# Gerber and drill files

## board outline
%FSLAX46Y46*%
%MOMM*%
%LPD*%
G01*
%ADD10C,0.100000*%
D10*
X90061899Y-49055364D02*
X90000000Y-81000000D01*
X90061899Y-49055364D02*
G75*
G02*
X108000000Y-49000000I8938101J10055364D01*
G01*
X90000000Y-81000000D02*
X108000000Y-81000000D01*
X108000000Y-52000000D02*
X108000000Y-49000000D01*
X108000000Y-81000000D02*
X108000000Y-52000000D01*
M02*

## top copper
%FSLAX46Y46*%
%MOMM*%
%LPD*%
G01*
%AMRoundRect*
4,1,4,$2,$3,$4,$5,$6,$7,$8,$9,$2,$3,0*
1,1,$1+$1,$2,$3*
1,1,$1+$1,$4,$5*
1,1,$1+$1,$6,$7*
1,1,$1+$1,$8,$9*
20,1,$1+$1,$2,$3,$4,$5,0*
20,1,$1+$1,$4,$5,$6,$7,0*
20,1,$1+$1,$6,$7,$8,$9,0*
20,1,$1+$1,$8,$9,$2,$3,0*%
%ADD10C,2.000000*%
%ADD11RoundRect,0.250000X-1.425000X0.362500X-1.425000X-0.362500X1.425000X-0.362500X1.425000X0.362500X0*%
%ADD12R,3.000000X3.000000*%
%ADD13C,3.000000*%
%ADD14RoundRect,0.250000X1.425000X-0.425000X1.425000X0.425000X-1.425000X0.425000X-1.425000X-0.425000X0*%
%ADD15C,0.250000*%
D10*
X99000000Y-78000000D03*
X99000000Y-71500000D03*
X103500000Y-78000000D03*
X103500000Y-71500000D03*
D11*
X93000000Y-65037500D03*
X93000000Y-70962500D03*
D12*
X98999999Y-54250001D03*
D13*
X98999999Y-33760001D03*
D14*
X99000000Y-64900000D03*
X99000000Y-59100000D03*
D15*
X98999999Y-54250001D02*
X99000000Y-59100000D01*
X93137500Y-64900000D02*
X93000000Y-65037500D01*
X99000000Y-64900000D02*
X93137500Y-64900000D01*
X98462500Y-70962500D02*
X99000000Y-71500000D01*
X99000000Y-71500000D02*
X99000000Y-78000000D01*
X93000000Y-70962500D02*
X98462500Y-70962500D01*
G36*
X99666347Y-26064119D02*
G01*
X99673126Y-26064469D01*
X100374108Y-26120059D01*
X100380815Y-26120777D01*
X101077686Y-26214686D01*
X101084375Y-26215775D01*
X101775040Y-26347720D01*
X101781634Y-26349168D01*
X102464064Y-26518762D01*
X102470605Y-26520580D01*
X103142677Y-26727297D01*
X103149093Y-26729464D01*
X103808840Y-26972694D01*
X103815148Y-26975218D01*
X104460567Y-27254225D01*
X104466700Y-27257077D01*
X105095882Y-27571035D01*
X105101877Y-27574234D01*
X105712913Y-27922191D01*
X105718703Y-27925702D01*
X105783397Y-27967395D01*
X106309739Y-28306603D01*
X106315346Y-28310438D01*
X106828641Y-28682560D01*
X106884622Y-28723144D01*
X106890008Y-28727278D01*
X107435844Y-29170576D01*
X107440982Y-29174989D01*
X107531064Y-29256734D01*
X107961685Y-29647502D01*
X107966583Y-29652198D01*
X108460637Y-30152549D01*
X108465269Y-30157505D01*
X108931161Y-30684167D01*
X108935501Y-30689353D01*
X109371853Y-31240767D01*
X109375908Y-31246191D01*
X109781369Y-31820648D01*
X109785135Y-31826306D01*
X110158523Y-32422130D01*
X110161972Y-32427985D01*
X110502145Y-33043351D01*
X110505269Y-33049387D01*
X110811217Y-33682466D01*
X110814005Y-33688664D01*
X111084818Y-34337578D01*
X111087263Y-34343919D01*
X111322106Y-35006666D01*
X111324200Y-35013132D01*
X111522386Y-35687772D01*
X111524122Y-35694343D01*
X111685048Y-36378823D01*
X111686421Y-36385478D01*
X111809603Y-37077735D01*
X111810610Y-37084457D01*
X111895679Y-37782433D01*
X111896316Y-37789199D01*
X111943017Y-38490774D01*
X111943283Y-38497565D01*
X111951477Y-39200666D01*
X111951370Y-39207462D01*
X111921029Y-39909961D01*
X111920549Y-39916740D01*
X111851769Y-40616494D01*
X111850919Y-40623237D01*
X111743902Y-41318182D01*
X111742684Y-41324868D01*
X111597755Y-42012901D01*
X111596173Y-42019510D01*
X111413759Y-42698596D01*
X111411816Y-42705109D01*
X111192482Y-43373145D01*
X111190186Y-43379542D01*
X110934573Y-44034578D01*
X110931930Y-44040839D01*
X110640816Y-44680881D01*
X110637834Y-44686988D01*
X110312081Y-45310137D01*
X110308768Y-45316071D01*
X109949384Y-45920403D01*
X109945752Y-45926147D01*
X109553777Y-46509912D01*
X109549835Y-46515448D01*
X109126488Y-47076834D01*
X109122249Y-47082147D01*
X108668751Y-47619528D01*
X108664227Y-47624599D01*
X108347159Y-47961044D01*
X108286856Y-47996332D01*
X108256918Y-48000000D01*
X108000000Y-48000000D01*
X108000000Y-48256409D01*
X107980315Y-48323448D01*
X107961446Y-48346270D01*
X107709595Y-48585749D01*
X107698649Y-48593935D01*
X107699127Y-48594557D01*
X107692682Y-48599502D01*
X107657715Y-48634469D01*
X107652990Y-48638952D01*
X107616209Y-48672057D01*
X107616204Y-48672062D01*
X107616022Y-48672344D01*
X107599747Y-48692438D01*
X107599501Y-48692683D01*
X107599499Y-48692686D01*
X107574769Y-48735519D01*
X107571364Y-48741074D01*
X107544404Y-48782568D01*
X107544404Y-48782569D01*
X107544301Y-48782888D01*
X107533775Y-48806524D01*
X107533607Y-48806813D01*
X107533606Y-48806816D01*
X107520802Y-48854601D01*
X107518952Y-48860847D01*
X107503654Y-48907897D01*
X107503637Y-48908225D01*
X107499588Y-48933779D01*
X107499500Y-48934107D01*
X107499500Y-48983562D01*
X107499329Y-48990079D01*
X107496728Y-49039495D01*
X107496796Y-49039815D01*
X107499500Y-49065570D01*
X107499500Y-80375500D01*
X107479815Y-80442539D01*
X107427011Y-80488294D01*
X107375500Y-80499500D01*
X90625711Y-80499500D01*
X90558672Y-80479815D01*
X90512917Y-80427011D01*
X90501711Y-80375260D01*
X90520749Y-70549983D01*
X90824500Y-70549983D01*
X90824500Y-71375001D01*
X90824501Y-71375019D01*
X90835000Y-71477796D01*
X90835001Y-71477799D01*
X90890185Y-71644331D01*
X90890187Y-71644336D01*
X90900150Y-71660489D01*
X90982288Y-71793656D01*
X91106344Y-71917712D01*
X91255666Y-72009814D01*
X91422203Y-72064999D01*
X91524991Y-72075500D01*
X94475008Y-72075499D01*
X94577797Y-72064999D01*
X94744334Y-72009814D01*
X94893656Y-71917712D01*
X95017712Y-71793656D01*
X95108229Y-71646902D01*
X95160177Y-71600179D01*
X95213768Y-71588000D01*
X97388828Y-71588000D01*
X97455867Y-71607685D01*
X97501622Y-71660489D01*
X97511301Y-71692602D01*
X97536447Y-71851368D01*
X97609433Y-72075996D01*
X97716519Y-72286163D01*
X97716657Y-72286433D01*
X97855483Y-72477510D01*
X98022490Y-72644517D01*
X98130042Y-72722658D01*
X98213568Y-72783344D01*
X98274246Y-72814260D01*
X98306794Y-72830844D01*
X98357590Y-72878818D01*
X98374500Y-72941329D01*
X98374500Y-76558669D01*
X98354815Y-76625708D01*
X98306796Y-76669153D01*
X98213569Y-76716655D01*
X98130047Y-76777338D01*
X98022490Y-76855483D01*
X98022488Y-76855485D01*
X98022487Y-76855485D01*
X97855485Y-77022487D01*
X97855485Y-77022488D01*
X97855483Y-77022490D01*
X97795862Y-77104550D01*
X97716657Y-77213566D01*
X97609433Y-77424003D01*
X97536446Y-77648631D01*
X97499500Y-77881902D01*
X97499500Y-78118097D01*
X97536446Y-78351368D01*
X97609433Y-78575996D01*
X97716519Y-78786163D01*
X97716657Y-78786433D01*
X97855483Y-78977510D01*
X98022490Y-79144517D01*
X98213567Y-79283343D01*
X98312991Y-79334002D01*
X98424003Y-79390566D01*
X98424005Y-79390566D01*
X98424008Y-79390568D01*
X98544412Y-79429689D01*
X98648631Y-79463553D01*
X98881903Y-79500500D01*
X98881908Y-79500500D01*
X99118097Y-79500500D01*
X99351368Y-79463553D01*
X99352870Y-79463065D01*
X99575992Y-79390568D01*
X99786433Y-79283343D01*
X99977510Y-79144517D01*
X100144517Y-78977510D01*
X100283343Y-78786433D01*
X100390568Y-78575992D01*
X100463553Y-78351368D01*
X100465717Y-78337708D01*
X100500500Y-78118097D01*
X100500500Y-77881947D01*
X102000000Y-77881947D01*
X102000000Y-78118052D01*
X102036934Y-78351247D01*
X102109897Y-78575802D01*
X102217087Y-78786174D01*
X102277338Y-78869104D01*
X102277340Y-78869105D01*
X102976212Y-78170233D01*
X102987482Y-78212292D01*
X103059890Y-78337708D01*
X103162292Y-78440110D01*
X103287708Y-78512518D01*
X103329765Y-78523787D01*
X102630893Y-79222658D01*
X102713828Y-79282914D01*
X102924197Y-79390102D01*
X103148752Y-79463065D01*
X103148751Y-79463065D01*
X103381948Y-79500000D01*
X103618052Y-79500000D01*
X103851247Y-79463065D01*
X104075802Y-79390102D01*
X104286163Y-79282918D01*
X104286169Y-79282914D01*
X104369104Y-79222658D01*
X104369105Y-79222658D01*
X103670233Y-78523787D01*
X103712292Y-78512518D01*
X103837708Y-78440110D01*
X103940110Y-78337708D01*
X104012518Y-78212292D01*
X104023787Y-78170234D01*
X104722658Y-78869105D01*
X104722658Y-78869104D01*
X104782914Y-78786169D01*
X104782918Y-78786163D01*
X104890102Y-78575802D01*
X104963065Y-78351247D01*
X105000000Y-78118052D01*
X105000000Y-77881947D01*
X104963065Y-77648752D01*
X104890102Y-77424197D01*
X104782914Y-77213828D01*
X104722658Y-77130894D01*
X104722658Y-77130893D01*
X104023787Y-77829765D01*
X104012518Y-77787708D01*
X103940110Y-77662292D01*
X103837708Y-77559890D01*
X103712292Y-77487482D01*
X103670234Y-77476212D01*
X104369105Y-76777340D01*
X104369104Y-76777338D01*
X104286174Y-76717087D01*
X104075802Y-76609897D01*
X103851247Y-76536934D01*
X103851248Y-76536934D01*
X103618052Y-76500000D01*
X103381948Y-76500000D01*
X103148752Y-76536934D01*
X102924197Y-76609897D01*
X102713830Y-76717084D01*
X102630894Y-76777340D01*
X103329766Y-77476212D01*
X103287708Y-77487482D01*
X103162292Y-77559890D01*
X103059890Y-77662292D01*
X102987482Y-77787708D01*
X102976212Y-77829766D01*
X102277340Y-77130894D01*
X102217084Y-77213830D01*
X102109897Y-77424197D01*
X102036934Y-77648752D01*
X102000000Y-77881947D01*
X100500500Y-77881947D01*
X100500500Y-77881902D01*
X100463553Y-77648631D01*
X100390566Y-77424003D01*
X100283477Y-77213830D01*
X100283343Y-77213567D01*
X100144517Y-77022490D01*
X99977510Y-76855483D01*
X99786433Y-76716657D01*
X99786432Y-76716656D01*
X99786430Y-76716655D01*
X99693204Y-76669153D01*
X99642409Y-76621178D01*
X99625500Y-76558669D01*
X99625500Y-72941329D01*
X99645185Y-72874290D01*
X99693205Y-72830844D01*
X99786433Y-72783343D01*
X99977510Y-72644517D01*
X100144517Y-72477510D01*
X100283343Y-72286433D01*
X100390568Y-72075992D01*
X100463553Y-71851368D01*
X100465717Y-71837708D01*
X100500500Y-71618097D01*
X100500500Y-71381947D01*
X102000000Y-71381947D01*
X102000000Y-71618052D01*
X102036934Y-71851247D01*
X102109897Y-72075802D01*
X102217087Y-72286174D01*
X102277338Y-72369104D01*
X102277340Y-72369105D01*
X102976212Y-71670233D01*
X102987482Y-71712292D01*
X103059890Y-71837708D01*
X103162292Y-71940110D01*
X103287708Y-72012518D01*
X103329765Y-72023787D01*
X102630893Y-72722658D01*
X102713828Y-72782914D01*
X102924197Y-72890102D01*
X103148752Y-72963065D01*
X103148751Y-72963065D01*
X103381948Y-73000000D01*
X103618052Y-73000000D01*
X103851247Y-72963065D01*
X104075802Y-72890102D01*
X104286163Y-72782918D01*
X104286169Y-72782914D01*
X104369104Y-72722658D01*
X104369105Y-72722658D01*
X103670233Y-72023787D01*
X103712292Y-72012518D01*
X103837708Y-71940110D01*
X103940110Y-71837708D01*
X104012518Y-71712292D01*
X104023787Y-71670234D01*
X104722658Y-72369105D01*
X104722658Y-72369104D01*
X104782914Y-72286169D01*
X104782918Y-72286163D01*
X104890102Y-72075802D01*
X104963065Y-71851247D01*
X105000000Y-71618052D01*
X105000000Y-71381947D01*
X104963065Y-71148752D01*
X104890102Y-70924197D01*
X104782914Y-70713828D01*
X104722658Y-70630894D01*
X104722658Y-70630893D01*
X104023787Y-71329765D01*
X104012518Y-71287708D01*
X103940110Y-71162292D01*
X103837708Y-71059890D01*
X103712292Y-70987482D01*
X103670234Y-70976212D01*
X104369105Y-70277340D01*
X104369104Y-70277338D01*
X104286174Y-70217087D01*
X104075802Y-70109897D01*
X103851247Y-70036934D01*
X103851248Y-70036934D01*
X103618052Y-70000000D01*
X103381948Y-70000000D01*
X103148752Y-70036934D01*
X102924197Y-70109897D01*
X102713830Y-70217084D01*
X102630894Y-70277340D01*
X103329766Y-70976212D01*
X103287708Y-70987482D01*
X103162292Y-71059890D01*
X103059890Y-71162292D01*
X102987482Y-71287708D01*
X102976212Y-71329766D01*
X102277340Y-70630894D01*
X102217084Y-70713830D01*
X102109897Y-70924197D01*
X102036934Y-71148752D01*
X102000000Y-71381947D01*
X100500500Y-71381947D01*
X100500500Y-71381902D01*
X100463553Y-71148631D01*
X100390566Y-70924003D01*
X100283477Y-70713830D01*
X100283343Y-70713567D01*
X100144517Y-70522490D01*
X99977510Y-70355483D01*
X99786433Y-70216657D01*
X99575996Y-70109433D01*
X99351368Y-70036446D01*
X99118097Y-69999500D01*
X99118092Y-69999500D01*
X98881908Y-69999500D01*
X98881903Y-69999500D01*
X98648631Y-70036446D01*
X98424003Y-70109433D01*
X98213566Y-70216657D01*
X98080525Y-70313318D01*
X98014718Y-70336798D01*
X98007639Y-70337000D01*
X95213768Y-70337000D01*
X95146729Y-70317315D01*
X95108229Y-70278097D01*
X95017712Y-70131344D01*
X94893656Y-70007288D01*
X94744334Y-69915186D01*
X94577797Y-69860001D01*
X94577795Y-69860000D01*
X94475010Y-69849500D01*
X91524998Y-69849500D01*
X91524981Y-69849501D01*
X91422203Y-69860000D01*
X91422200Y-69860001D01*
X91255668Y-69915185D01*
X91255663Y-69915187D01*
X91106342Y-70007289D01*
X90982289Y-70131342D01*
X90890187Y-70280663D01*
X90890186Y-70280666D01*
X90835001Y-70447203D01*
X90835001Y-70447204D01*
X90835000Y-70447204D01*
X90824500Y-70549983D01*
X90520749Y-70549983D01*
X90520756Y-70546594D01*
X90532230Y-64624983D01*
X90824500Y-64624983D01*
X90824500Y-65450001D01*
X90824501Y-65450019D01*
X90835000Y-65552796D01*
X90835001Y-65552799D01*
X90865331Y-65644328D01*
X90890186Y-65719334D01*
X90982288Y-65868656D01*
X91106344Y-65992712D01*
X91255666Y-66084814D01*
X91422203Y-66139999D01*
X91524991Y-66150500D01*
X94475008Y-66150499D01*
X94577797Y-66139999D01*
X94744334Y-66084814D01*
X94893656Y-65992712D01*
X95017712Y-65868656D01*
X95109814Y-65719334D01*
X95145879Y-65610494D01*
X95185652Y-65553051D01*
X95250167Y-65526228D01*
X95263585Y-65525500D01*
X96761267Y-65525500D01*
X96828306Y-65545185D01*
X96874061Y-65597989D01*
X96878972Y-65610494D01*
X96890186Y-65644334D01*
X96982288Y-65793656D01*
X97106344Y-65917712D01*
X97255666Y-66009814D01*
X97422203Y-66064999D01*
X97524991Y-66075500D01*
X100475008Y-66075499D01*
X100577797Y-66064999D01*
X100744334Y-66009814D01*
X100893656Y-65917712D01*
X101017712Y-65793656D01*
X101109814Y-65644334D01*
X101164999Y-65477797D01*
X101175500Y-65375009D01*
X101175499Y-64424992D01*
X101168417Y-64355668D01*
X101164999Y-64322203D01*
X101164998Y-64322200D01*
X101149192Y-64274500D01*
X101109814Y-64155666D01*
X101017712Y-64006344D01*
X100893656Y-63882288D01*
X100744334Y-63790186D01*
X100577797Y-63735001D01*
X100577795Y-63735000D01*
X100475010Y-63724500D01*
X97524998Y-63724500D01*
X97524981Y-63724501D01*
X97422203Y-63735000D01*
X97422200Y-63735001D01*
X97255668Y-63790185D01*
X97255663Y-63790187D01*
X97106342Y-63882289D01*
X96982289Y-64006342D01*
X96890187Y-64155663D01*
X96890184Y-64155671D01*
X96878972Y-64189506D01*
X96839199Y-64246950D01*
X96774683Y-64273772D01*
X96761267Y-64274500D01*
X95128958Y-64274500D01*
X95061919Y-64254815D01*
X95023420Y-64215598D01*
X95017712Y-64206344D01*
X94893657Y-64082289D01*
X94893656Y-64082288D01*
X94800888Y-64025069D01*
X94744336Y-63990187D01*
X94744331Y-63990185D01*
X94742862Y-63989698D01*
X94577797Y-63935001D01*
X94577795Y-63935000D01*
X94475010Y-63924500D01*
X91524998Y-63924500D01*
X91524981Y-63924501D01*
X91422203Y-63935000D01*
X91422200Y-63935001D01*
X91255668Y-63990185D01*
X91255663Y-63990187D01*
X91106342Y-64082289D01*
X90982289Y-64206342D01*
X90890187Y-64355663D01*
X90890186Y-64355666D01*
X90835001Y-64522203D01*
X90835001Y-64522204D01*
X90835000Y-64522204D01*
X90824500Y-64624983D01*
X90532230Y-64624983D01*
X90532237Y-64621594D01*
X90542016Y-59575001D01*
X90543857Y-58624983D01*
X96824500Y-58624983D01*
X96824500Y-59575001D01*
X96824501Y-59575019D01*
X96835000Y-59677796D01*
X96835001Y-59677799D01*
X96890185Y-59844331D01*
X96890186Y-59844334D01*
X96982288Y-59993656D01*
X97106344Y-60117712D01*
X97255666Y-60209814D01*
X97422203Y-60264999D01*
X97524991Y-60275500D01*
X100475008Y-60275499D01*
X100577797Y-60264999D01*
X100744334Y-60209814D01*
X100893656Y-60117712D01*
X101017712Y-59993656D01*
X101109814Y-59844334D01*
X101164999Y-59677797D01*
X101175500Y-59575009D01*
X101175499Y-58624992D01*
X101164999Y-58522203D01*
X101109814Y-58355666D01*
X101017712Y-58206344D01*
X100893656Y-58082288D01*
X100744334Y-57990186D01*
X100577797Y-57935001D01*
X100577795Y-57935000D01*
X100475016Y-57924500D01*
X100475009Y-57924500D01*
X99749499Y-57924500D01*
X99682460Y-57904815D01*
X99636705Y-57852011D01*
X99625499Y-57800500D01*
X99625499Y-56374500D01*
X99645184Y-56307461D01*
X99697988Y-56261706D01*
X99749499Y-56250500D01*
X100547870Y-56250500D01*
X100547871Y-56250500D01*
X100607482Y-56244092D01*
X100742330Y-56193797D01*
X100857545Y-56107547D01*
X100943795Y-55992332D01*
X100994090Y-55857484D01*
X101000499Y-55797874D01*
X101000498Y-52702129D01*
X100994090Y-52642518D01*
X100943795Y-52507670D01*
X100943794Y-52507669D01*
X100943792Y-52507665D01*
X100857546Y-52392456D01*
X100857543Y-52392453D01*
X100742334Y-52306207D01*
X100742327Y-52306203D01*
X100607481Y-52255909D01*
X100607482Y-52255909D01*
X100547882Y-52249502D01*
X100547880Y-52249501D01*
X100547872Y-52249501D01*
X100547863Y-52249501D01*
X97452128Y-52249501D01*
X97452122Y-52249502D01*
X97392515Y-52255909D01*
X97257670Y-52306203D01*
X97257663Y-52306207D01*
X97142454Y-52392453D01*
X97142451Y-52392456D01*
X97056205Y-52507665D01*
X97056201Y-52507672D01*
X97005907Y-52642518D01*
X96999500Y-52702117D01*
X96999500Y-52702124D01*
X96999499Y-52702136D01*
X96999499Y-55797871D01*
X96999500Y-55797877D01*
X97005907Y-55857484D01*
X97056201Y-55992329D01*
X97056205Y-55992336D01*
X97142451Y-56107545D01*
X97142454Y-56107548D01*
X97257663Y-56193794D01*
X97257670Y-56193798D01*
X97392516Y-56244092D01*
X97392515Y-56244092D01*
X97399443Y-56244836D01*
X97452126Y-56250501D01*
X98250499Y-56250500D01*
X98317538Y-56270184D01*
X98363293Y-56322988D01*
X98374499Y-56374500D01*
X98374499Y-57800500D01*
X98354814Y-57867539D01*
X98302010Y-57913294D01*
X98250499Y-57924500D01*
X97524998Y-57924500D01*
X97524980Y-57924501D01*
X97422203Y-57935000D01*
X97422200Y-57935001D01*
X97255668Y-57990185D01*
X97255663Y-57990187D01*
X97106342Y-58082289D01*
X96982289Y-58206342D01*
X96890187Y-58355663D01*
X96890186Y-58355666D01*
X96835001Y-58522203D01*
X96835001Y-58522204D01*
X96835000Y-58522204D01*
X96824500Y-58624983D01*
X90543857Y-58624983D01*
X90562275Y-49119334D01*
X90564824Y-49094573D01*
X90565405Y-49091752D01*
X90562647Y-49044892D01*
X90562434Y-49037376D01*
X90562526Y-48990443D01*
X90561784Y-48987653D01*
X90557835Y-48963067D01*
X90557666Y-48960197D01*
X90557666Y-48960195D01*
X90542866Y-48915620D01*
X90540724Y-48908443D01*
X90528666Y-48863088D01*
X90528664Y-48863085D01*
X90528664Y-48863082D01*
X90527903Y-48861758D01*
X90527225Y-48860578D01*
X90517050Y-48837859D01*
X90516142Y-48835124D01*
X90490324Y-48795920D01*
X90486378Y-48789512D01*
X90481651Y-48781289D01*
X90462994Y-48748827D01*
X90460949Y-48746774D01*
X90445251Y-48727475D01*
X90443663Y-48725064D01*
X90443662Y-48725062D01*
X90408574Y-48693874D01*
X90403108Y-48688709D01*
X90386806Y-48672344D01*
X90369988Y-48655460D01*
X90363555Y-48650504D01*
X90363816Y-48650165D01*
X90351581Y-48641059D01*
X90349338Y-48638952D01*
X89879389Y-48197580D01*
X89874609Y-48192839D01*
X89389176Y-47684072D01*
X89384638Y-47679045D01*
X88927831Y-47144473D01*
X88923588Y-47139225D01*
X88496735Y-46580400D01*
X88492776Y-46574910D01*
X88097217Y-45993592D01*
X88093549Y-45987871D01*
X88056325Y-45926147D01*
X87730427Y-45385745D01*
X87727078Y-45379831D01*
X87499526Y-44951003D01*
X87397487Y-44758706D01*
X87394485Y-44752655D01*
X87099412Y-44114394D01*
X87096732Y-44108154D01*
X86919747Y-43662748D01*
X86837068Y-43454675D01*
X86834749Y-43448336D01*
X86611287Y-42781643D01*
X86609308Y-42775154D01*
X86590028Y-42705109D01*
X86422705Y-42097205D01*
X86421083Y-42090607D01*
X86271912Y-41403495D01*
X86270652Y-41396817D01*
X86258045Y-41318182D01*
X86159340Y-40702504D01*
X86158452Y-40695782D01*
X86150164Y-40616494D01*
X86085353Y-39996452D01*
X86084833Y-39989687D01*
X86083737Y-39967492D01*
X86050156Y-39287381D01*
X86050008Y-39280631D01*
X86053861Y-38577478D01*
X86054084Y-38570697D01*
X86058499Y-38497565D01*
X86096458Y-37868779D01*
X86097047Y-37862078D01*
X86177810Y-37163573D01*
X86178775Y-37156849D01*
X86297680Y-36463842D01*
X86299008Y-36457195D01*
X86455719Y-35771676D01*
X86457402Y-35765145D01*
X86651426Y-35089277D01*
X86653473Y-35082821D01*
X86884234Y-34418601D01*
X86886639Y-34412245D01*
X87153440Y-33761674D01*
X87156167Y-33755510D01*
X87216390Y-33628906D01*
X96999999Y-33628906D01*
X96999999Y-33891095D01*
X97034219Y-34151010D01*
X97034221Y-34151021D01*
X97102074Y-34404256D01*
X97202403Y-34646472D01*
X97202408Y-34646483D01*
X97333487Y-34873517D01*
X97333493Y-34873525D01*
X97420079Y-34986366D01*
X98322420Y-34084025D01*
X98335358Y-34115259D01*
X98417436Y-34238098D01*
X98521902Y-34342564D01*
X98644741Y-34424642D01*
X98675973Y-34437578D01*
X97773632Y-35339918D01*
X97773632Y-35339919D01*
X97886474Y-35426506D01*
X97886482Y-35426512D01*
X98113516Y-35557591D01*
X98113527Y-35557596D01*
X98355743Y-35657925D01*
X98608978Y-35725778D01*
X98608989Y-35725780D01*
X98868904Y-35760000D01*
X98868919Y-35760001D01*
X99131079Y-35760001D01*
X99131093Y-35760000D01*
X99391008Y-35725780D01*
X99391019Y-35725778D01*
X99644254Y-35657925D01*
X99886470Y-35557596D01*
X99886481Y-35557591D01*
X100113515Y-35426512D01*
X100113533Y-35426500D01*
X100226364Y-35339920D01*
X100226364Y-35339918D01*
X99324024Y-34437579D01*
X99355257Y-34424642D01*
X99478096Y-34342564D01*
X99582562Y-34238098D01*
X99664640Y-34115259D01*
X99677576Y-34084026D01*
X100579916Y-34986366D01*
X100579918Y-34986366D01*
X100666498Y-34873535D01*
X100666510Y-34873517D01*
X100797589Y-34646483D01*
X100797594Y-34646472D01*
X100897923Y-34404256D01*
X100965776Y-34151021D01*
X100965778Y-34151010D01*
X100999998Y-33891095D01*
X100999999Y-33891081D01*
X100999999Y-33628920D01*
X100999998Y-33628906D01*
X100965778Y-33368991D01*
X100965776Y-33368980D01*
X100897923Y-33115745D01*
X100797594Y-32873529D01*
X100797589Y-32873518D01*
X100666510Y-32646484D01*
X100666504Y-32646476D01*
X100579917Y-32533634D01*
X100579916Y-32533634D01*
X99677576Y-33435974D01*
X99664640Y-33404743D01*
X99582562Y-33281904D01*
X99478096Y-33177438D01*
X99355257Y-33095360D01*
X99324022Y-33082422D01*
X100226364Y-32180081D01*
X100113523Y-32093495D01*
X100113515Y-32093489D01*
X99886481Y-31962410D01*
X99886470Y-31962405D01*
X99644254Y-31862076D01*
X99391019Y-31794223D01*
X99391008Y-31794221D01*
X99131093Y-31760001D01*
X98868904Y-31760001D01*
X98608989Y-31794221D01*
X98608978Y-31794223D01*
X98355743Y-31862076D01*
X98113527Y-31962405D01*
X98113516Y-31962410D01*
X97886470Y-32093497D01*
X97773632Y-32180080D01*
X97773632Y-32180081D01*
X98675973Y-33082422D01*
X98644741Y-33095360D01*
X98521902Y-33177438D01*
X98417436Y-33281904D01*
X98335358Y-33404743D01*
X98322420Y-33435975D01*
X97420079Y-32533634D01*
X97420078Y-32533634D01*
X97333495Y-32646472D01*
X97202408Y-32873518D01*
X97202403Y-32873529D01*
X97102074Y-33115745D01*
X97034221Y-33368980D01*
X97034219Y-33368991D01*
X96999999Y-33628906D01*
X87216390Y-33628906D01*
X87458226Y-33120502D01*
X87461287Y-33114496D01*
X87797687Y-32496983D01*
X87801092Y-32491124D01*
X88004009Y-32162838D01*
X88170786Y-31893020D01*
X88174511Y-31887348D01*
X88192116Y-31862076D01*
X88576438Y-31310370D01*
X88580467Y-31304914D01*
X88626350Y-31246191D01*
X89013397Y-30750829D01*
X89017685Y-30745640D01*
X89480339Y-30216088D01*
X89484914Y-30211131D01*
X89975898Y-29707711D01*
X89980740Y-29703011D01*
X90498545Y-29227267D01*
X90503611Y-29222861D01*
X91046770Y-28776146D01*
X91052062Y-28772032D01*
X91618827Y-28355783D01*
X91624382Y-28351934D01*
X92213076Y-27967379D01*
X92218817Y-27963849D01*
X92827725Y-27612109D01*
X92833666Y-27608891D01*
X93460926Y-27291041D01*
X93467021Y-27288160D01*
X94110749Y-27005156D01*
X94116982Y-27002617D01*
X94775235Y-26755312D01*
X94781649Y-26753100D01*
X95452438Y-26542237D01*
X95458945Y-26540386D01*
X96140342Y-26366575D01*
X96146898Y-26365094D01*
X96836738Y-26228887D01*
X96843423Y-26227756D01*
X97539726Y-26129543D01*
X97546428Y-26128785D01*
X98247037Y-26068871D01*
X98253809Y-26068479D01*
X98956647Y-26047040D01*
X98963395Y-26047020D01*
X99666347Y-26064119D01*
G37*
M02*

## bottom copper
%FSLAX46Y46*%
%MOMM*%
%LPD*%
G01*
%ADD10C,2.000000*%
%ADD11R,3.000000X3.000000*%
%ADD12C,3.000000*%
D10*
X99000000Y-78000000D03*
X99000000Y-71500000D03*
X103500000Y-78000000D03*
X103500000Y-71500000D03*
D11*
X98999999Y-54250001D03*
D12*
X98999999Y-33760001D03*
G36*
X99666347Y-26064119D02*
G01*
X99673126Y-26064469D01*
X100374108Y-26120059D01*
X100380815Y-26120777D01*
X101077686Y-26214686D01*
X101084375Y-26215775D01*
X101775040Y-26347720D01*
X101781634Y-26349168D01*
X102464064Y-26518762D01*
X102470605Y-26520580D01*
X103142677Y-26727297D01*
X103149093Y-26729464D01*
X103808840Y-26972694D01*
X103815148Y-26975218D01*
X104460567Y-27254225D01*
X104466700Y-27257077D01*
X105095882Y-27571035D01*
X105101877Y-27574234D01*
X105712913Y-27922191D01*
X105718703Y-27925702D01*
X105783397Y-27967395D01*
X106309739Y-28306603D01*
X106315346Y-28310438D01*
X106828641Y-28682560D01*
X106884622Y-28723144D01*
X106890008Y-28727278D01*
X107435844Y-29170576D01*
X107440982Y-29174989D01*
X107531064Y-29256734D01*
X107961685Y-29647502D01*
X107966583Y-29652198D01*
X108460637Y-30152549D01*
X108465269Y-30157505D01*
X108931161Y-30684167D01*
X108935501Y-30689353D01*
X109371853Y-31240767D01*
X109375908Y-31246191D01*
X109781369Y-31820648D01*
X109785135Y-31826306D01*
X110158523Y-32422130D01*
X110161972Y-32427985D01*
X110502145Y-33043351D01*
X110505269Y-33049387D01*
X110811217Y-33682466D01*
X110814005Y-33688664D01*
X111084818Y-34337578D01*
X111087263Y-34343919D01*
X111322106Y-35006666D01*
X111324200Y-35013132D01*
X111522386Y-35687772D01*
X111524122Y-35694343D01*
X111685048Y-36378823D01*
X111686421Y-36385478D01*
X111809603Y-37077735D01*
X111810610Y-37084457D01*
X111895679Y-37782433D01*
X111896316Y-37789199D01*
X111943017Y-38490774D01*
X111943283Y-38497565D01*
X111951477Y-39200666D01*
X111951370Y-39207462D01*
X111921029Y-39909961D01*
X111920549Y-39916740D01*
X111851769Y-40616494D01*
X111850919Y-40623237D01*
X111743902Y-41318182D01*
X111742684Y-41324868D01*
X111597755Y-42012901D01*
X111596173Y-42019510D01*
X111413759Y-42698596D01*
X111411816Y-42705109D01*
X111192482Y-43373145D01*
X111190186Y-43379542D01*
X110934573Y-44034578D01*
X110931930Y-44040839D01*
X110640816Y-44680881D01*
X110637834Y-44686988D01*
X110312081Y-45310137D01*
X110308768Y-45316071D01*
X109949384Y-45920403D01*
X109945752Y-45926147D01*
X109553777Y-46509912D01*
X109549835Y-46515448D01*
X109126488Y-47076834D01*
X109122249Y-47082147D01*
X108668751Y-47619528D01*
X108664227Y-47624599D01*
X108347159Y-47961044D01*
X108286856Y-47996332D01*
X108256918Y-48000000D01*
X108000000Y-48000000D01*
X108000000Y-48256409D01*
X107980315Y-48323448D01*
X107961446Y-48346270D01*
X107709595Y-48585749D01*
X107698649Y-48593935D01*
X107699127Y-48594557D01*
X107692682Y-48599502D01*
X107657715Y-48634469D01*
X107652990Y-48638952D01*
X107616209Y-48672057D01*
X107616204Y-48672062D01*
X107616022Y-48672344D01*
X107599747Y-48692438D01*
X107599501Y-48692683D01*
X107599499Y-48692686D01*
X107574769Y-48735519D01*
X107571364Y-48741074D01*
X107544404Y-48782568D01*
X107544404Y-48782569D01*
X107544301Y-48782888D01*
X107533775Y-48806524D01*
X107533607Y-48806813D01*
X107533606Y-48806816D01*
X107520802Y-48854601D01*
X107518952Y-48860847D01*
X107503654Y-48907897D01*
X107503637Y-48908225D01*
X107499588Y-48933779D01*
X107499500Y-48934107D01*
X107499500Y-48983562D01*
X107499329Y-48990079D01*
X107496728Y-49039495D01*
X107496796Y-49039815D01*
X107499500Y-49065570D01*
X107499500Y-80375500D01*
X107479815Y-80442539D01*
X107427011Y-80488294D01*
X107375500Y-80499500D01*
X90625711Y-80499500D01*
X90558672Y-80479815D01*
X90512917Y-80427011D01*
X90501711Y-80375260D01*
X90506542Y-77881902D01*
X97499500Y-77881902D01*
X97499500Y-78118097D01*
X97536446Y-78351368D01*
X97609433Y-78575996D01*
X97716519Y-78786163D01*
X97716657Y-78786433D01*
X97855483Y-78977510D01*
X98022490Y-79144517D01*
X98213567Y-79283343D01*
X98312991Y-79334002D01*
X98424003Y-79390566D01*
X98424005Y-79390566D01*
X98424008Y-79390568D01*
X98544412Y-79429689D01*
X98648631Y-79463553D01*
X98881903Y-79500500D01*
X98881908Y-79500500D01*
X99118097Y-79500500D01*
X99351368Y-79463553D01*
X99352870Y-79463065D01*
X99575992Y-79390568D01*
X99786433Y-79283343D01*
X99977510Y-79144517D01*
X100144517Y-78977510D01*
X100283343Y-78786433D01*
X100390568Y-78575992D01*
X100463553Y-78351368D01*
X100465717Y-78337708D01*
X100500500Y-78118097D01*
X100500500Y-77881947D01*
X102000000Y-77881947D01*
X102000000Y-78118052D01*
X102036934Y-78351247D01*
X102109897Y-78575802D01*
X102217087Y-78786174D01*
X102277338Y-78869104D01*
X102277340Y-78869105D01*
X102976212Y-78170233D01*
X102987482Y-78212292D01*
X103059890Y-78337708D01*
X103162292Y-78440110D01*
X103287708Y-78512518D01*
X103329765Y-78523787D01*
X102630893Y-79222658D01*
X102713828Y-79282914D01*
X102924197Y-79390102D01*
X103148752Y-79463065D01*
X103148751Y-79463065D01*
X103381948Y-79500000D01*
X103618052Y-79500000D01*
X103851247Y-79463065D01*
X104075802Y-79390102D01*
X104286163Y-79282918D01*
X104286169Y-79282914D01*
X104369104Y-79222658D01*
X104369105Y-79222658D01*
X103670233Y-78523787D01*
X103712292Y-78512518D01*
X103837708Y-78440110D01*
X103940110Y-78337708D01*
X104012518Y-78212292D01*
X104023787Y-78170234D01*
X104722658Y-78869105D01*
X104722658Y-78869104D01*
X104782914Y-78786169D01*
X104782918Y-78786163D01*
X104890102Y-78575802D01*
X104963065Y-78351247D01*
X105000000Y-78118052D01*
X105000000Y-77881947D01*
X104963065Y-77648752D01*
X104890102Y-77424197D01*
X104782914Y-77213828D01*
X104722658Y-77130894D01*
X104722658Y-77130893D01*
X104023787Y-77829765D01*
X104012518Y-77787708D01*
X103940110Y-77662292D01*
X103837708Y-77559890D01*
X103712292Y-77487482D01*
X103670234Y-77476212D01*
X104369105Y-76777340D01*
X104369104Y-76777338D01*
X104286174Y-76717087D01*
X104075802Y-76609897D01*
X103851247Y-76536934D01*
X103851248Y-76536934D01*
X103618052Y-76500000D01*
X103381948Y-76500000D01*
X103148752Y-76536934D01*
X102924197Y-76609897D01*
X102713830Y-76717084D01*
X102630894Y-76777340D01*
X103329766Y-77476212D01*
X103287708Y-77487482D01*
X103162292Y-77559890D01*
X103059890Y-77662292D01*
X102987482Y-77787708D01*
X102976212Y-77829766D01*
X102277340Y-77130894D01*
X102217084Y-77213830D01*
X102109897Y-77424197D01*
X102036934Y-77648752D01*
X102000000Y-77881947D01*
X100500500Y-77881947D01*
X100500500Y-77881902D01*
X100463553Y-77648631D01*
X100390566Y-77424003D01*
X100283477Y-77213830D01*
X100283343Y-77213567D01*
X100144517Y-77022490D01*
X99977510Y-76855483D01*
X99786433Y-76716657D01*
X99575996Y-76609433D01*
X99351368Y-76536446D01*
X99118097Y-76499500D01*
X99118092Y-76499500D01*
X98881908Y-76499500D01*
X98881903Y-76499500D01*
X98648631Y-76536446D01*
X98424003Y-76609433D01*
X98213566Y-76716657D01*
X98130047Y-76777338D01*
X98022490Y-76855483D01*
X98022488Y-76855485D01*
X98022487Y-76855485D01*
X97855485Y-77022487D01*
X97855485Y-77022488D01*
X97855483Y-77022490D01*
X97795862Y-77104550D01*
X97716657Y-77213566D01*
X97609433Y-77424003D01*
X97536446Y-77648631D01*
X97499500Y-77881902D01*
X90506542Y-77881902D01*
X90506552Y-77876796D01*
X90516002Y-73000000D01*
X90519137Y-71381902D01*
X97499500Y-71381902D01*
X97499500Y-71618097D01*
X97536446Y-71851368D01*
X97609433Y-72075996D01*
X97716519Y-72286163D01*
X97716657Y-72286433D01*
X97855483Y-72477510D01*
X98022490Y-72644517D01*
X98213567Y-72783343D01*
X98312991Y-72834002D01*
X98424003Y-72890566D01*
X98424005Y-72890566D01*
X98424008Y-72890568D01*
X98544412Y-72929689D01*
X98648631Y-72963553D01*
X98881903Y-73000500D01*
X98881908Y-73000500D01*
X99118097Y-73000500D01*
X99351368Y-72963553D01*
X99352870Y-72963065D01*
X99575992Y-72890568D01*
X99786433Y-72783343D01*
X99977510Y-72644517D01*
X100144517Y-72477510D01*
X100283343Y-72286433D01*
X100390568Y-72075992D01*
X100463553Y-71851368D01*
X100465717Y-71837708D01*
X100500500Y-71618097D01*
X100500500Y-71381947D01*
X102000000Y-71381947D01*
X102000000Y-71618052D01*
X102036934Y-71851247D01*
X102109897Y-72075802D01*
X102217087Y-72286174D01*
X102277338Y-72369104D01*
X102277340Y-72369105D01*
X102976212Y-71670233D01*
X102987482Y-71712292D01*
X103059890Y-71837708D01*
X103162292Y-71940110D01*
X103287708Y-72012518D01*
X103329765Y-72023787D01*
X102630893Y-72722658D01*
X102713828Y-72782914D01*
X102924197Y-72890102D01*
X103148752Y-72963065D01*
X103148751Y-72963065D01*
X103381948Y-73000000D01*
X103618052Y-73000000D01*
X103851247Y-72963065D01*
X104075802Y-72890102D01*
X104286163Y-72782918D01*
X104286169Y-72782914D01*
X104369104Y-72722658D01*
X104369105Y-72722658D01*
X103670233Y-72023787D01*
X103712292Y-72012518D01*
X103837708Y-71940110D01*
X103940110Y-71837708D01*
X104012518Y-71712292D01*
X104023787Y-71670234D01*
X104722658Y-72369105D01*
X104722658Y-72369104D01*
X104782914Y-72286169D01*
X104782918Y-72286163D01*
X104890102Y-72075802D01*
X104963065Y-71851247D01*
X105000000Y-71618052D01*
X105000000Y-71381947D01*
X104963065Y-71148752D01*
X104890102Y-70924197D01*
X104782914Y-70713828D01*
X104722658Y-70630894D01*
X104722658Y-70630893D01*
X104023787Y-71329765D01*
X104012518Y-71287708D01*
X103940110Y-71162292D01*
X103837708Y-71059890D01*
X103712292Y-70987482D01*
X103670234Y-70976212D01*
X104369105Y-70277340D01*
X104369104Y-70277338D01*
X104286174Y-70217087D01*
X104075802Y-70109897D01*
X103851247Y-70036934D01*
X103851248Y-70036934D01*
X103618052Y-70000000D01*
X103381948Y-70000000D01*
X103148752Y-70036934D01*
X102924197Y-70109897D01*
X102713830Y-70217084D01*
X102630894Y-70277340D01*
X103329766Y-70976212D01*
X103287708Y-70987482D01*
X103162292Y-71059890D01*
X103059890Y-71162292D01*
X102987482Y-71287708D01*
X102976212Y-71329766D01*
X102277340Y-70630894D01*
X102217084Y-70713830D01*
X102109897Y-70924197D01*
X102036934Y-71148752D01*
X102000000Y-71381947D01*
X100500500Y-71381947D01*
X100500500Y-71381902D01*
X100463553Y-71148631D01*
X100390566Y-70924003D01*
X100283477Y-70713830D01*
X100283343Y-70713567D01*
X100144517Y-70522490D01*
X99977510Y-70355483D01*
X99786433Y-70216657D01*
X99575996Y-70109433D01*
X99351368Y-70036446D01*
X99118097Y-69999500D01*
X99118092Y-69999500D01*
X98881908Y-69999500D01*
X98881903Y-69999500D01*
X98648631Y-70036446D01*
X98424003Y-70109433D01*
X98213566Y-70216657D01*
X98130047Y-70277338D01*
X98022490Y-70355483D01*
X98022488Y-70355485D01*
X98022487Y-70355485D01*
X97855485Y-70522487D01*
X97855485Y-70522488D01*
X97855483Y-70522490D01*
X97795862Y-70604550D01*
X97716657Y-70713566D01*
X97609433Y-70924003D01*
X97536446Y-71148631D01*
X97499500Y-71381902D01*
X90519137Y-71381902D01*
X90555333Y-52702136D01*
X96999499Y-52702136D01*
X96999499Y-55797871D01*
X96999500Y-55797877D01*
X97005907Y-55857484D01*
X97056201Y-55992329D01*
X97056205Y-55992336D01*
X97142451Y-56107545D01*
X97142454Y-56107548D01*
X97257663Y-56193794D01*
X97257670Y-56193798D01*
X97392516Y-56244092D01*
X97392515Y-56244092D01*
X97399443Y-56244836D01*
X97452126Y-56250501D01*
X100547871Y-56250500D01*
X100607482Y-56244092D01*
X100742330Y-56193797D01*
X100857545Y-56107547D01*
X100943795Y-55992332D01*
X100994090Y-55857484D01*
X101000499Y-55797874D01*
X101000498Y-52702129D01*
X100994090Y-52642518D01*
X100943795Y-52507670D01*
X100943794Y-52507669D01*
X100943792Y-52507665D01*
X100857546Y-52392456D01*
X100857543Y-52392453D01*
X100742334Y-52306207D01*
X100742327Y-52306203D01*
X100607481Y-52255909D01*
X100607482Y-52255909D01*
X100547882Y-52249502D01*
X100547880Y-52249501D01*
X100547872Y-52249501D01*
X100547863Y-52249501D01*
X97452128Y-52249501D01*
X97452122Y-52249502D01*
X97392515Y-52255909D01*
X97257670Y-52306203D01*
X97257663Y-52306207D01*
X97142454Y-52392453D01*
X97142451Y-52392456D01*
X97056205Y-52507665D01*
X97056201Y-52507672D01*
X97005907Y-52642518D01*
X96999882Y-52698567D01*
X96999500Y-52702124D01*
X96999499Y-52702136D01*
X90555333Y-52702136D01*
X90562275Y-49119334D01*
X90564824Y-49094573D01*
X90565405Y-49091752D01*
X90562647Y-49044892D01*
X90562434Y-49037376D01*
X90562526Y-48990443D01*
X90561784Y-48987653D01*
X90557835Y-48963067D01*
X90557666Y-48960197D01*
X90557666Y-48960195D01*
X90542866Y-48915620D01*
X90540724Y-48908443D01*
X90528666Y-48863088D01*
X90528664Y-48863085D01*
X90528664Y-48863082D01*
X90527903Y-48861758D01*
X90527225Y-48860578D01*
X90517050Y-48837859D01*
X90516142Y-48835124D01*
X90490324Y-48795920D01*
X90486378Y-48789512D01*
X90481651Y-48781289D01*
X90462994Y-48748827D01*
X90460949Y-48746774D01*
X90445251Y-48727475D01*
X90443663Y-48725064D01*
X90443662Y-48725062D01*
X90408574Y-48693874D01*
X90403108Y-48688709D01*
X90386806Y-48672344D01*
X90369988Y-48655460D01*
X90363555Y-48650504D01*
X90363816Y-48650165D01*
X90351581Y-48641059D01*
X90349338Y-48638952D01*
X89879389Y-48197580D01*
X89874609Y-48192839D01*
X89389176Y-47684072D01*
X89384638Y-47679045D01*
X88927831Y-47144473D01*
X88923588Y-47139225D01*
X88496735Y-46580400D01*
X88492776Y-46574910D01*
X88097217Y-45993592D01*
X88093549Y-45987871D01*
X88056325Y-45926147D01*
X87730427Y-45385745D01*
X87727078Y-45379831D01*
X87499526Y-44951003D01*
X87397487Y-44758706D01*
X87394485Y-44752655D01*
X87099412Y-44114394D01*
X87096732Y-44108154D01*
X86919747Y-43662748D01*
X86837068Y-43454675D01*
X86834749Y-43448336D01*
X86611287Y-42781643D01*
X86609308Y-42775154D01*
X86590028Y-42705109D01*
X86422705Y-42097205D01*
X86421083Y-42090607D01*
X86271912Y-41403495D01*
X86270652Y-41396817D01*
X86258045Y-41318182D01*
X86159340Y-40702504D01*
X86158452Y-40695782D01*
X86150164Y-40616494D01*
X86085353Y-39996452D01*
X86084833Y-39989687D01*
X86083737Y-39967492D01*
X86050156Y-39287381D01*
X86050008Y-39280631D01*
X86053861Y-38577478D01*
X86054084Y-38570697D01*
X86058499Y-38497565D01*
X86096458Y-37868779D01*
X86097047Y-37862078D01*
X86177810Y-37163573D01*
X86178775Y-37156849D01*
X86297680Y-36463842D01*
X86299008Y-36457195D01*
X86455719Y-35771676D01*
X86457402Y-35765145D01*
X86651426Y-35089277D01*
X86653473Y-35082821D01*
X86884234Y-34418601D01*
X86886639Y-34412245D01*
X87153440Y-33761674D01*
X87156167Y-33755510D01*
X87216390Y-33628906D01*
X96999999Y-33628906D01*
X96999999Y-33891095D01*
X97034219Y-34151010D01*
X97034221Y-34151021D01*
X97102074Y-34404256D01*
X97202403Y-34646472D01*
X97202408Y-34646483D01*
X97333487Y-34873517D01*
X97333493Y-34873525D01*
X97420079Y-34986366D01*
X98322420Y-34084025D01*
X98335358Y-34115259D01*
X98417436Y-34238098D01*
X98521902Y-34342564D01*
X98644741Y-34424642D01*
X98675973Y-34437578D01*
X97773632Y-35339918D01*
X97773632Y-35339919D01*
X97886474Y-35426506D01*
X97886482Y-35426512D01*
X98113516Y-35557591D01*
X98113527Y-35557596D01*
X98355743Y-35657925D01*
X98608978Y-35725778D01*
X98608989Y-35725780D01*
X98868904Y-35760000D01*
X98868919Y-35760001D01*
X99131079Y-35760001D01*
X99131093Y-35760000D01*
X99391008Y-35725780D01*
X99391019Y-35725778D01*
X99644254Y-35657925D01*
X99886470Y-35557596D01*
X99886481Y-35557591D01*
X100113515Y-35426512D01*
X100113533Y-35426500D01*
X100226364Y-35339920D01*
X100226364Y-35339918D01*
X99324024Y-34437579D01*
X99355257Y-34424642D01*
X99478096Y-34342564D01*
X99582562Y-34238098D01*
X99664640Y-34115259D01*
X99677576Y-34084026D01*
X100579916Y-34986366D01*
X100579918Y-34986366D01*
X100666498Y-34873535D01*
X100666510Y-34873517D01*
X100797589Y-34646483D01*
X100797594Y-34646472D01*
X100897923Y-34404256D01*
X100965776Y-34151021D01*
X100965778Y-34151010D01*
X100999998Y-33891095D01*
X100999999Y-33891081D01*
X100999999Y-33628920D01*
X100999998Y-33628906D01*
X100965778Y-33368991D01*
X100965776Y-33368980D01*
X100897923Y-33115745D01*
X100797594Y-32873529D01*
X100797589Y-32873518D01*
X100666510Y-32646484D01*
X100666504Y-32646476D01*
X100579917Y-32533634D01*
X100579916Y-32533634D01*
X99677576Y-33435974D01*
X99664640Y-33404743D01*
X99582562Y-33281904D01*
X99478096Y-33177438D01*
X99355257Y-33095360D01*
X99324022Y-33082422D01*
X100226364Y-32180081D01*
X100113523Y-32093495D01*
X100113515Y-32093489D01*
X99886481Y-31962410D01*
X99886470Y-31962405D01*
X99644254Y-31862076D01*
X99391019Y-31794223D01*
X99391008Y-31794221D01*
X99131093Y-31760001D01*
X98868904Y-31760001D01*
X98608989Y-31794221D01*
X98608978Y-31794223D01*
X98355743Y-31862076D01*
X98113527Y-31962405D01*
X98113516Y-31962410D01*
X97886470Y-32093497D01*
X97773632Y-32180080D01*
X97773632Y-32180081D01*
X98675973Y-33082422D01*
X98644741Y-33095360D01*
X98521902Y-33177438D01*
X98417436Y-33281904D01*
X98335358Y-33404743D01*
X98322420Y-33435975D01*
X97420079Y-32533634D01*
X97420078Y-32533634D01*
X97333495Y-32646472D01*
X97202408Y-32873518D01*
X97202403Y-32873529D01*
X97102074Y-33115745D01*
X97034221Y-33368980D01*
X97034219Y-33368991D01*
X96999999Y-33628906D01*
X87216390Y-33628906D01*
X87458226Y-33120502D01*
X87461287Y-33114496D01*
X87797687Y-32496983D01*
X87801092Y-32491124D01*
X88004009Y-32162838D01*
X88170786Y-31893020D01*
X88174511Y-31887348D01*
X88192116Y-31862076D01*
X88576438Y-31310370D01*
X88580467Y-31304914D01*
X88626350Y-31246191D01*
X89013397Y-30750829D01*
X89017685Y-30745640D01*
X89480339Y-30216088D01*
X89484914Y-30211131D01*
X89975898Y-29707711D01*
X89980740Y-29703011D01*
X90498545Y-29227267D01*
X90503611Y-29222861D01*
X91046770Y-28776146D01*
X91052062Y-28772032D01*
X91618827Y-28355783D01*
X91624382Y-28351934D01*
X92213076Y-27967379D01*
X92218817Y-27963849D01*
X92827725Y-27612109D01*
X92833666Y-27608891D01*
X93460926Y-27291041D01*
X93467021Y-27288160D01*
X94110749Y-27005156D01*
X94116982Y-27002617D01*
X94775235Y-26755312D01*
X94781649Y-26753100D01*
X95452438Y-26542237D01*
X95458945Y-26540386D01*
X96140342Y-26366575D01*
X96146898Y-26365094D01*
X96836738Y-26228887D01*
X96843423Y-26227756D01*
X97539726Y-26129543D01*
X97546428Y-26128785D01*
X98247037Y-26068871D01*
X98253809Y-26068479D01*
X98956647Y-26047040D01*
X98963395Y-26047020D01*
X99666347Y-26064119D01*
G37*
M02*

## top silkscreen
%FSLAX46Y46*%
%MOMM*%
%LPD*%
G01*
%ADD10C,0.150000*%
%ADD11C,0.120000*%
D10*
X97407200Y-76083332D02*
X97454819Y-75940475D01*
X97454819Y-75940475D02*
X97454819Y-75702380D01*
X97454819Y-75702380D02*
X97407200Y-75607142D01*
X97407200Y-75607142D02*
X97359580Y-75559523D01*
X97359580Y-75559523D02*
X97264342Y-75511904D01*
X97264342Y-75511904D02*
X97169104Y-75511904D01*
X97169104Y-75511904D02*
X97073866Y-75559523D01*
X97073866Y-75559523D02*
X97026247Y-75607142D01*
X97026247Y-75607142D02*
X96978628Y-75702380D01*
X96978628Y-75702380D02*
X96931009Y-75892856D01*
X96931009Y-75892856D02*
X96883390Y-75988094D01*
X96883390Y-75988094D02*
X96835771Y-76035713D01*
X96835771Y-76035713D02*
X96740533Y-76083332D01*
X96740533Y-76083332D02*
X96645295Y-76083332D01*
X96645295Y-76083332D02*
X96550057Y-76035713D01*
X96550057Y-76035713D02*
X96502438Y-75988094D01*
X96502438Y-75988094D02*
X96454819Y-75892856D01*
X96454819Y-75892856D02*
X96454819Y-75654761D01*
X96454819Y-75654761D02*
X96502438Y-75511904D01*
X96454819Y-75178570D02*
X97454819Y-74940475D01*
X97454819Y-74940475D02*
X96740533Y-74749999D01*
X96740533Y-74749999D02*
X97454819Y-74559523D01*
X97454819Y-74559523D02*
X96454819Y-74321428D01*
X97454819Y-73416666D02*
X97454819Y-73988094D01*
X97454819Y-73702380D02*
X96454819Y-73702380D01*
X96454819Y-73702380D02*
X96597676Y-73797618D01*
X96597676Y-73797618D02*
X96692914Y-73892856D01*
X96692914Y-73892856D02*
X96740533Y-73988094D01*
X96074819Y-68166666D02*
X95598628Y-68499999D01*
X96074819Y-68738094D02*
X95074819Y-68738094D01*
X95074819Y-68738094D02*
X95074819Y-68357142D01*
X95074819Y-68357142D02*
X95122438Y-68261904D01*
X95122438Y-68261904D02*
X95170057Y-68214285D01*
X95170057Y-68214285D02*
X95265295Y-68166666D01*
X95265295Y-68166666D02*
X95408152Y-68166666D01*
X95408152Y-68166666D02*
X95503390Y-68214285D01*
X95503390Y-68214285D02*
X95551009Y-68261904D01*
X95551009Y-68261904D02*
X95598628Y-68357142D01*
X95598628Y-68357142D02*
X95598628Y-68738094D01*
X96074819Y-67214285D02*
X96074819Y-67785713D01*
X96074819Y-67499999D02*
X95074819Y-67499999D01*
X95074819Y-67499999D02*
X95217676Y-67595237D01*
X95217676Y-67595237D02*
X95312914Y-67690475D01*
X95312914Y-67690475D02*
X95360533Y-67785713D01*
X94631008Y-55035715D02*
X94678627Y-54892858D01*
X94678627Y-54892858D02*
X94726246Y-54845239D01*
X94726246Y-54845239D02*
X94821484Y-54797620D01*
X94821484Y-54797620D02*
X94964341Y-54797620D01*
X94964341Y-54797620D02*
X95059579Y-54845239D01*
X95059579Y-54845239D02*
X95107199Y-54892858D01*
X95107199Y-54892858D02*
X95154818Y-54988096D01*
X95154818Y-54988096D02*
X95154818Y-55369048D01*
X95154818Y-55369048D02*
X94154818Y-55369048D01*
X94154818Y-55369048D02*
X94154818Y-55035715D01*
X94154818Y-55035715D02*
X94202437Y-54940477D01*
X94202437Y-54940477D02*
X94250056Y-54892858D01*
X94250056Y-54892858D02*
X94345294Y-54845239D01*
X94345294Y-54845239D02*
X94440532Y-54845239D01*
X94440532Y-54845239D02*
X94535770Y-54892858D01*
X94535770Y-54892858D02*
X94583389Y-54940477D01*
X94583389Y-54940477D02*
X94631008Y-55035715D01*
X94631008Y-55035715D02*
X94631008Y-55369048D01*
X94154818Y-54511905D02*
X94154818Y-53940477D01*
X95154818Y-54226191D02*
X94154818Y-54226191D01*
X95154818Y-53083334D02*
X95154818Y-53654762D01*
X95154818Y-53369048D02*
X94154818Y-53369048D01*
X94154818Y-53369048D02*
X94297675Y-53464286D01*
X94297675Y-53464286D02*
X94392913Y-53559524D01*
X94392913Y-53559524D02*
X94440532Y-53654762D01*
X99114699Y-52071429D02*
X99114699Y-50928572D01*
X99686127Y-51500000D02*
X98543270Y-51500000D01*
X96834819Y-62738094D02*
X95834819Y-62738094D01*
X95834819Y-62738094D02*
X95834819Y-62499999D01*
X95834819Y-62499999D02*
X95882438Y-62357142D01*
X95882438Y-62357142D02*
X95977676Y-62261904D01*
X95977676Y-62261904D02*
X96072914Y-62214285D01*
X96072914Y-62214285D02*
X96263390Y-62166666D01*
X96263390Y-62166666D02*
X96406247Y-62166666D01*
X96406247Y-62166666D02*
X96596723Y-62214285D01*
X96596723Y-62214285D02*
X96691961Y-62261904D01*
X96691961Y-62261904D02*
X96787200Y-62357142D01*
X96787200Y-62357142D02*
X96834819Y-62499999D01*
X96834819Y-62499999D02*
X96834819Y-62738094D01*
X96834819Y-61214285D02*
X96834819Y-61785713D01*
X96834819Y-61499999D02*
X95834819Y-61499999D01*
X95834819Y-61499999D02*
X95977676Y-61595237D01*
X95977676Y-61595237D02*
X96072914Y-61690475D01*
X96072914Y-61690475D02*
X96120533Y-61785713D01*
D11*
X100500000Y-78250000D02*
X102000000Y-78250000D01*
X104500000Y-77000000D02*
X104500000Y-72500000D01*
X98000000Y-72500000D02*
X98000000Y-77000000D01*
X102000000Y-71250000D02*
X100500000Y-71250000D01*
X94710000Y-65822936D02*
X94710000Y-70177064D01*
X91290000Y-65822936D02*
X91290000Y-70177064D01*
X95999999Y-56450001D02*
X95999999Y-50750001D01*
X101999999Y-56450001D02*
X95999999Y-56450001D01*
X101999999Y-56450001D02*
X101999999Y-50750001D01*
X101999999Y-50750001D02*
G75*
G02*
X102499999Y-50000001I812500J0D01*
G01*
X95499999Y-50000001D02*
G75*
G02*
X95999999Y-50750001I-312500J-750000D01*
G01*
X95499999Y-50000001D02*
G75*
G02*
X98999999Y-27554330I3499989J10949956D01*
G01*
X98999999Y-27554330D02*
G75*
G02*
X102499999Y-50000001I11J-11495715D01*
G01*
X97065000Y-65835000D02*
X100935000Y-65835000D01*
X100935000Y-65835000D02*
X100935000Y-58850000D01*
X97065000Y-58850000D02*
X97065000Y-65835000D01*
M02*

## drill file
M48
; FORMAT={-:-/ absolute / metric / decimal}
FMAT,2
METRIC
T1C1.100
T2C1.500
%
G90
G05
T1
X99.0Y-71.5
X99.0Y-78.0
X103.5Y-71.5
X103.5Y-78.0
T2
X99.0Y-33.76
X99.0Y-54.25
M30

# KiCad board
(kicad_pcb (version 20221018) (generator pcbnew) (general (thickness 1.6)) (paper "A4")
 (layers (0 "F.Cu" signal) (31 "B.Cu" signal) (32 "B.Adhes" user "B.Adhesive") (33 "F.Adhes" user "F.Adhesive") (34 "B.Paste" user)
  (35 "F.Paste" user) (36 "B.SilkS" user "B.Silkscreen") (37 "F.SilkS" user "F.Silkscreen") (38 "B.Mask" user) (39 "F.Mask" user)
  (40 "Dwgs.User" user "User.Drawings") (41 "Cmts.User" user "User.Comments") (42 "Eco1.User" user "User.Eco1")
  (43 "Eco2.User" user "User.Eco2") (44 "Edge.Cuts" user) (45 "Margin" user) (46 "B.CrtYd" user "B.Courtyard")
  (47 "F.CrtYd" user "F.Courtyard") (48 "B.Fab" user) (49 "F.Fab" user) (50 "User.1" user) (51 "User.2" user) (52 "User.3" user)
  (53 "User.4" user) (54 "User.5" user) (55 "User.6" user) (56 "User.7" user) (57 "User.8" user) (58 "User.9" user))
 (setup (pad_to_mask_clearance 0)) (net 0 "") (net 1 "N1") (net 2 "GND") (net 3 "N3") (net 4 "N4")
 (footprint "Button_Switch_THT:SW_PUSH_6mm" (layer "F.Cu") (at 99 78 90)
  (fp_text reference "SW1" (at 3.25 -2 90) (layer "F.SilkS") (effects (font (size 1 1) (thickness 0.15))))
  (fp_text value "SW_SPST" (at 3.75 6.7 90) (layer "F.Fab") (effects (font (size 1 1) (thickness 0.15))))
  (fp_line (start -0.25 1.5) (end -0.25 3) (stroke (width 0.12) (type solid)) (layer "F.SilkS"))
  (fp_line (start 1 5.5) (end 5.5 5.5) (stroke (width 0.12) (type solid)) (layer "F.SilkS"))
  (fp_line (start 5.5 -1) (end 1 -1) (stroke (width 0.12) (type solid)) (layer "F.SilkS"))
  (fp_line (start 6.75 3) (end 6.75 1.5) (stroke (width 0.12) (type solid)) (layer "F.SilkS"))
  (pad "1" thru_hole circle (at 0 0 180) (size 2 2) (drill 1.1) (layers "*.Cu" "*.Mask") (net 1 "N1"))
  (pad "1" thru_hole circle (at 6.5 0 180) (size 2 2) (drill 1.1) (layers "*.Cu" "*.Mask") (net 1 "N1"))
  (pad "2" thru_hole circle (at 0 4.5 180) (size 2 2) (drill 1.1) (layers "*.Cu" "*.Mask") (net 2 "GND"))
  (pad "2" thru_hole circle (at 6.5 4.5 180) (size 2 2) (drill 1.1) (layers "*.Cu" "*.Mask") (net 2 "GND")))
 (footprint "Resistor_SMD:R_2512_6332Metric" (layer "F.Cu") (at 93 68 -90)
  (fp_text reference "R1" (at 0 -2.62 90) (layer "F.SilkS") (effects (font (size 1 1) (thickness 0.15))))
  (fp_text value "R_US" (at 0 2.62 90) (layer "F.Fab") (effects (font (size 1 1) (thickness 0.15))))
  (fp_line (start -2.177064 -1.71) (end 2.177064 -1.71) (stroke (width 0.12) (type solid)) (layer "F.SilkS"))
  (fp_line (start -2.177064 1.71) (end 2.177064 1.71) (stroke (width 0.12) (type solid)) (layer "F.SilkS"))
  (pad "1" smd roundrect (at -2.9625 0 270) (size 1.225 3.35) (layers "F.Cu" "F.Paste" "F.Mask") (roundrect_rratio 0.204082) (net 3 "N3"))
  (pad "2" smd roundrect (at 2.9625 0 270) (size 1.225 3.35) (layers "F.Cu" "F.Paste" "F.Mask") (roundrect_rratio 0.204082) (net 1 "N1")))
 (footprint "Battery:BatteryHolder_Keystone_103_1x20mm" (layer "F.Cu") (at 98.999999 54.250001 90)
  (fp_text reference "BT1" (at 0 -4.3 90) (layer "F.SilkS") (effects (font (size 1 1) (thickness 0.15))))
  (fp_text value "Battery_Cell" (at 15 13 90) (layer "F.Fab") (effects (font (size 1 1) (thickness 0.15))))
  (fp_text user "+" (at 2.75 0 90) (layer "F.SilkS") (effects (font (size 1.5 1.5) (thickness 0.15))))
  (fp_line (start -2.2 -3) (end 3.5 -3) (stroke (width 0.12) (type solid)) (layer "F.SilkS"))
  (fp_line (start -2.2 3) (end -2.2 -3) (stroke (width 0.12) (type solid)) (layer "F.SilkS"))
  (fp_line (start -2.2 3) (end 3.5 3) (stroke (width 0.12) (type solid)) (layer "F.SilkS"))
  (fp_arc (start 3.5 3) (mid 3.950694 3.136459) (end 4.25 3.5) (stroke (width 0.12) (type solid)) (layer "F.SilkS"))
  (fp_arc (start 4.25 -3.5) (mid 3.950694 -3.136459) (end 3.5 -3) (stroke (width 0.12) (type solid)) (layer "F.SilkS"))
  (fp_arc (start 4.25 -3.5) (mid 16.971103 -11.358466) (end 26.695671 0) (stroke (width 0.12) (type solid)) (layer "F.SilkS"))
  (fp_arc (start 26.695671 0) (mid 16.971103 11.358466) (end 4.25 3.5) (stroke (width 0.12) (type solid)) (layer "F.SilkS"))
  (pad "1" thru_hole rect (at 0 0 90) (size 3 3) (drill 1.5) (layers "*.Cu" "*.Mask") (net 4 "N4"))
  (pad "2" thru_hole circle (at 20.49 0 90) (size 3 3) (drill 1.5) (layers "*.Cu" "*.Mask") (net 2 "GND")))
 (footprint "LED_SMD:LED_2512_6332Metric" (layer "F.Cu") (at 99 62 90)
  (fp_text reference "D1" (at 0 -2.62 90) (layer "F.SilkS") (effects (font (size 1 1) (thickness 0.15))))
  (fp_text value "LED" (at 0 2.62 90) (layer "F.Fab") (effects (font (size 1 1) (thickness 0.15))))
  (fp_line (start -3.835 -1.935) (end -3.835 1.935) (stroke (width 0.12) (type solid)) (layer "F.SilkS"))
  (fp_line (start -3.835 1.935) (end 3.15 1.935) (stroke (width 0.12) (type solid)) (layer "F.SilkS"))
  (fp_line (start 3.15 -1.935) (end -3.835 -1.935) (stroke (width 0.12) (type solid)) (layer "F.SilkS"))
  (pad "1" smd roundrect (at -2.9 0 90) (size 1.35 3.35) (layers "F.Cu" "F.Paste" "F.Mask") (roundrect_rratio 0.185185) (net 3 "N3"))
  (pad "2" smd roundrect (at 2.9 0 90) (size 1.35 3.35) (layers "F.Cu" "F.Paste" "F.Mask") (roundrect_rratio 0.185185) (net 4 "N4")))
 (gr_line (start 90.061899 49.055364) (end 90 81) (stroke (width 0.1) (type default)) (layer "Edge.Cuts"))
 (gr_arc (start 90.061899 49.055364) (mid 98.958477 25.54644) (end 108 49) (stroke (width 0.1) (type default)) (layer "Edge.Cuts"))
 (gr_line (start 90 81) (end 108 81) (stroke (width 0.1) (type default)) (layer "Edge.Cuts"))
 (gr_line (start 108 52) (end 108 49) (stroke (width 0.1) (type default)) (layer "Edge.Cuts"))
 (gr_line (start 108 81) (end 108 52) (stroke (width 0.1) (type default)) (layer "Edge.Cuts"))
 (segment (start 98.999999 54.250001) (end 99 59.1) (width 0.25) (layer "F.Cu") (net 4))
 (segment (start 93.1375 64.9) (end 93 65.0375) (width 0.25) (layer "F.Cu") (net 3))
 (segment (start 99 64.9) (end 93.1375 64.9) (width 0.25) (layer "F.Cu") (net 3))
 (segment (start 98.4625 70.9625) (end 99 71.5) (width 0.25) (layer "F.Cu") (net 1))
 (segment (start 99 71.5) (end 99 78) (width 0.25) (layer "F.Cu") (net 1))
 (segment (start 93 70.9625) (end 98.4625 70.9625) (width 0.25) (layer "F.Cu") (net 1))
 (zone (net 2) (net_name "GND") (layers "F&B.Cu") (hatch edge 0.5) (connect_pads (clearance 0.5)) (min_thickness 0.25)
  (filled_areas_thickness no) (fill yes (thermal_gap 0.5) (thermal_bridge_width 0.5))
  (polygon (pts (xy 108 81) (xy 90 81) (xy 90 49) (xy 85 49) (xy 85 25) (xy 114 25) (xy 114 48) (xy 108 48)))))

